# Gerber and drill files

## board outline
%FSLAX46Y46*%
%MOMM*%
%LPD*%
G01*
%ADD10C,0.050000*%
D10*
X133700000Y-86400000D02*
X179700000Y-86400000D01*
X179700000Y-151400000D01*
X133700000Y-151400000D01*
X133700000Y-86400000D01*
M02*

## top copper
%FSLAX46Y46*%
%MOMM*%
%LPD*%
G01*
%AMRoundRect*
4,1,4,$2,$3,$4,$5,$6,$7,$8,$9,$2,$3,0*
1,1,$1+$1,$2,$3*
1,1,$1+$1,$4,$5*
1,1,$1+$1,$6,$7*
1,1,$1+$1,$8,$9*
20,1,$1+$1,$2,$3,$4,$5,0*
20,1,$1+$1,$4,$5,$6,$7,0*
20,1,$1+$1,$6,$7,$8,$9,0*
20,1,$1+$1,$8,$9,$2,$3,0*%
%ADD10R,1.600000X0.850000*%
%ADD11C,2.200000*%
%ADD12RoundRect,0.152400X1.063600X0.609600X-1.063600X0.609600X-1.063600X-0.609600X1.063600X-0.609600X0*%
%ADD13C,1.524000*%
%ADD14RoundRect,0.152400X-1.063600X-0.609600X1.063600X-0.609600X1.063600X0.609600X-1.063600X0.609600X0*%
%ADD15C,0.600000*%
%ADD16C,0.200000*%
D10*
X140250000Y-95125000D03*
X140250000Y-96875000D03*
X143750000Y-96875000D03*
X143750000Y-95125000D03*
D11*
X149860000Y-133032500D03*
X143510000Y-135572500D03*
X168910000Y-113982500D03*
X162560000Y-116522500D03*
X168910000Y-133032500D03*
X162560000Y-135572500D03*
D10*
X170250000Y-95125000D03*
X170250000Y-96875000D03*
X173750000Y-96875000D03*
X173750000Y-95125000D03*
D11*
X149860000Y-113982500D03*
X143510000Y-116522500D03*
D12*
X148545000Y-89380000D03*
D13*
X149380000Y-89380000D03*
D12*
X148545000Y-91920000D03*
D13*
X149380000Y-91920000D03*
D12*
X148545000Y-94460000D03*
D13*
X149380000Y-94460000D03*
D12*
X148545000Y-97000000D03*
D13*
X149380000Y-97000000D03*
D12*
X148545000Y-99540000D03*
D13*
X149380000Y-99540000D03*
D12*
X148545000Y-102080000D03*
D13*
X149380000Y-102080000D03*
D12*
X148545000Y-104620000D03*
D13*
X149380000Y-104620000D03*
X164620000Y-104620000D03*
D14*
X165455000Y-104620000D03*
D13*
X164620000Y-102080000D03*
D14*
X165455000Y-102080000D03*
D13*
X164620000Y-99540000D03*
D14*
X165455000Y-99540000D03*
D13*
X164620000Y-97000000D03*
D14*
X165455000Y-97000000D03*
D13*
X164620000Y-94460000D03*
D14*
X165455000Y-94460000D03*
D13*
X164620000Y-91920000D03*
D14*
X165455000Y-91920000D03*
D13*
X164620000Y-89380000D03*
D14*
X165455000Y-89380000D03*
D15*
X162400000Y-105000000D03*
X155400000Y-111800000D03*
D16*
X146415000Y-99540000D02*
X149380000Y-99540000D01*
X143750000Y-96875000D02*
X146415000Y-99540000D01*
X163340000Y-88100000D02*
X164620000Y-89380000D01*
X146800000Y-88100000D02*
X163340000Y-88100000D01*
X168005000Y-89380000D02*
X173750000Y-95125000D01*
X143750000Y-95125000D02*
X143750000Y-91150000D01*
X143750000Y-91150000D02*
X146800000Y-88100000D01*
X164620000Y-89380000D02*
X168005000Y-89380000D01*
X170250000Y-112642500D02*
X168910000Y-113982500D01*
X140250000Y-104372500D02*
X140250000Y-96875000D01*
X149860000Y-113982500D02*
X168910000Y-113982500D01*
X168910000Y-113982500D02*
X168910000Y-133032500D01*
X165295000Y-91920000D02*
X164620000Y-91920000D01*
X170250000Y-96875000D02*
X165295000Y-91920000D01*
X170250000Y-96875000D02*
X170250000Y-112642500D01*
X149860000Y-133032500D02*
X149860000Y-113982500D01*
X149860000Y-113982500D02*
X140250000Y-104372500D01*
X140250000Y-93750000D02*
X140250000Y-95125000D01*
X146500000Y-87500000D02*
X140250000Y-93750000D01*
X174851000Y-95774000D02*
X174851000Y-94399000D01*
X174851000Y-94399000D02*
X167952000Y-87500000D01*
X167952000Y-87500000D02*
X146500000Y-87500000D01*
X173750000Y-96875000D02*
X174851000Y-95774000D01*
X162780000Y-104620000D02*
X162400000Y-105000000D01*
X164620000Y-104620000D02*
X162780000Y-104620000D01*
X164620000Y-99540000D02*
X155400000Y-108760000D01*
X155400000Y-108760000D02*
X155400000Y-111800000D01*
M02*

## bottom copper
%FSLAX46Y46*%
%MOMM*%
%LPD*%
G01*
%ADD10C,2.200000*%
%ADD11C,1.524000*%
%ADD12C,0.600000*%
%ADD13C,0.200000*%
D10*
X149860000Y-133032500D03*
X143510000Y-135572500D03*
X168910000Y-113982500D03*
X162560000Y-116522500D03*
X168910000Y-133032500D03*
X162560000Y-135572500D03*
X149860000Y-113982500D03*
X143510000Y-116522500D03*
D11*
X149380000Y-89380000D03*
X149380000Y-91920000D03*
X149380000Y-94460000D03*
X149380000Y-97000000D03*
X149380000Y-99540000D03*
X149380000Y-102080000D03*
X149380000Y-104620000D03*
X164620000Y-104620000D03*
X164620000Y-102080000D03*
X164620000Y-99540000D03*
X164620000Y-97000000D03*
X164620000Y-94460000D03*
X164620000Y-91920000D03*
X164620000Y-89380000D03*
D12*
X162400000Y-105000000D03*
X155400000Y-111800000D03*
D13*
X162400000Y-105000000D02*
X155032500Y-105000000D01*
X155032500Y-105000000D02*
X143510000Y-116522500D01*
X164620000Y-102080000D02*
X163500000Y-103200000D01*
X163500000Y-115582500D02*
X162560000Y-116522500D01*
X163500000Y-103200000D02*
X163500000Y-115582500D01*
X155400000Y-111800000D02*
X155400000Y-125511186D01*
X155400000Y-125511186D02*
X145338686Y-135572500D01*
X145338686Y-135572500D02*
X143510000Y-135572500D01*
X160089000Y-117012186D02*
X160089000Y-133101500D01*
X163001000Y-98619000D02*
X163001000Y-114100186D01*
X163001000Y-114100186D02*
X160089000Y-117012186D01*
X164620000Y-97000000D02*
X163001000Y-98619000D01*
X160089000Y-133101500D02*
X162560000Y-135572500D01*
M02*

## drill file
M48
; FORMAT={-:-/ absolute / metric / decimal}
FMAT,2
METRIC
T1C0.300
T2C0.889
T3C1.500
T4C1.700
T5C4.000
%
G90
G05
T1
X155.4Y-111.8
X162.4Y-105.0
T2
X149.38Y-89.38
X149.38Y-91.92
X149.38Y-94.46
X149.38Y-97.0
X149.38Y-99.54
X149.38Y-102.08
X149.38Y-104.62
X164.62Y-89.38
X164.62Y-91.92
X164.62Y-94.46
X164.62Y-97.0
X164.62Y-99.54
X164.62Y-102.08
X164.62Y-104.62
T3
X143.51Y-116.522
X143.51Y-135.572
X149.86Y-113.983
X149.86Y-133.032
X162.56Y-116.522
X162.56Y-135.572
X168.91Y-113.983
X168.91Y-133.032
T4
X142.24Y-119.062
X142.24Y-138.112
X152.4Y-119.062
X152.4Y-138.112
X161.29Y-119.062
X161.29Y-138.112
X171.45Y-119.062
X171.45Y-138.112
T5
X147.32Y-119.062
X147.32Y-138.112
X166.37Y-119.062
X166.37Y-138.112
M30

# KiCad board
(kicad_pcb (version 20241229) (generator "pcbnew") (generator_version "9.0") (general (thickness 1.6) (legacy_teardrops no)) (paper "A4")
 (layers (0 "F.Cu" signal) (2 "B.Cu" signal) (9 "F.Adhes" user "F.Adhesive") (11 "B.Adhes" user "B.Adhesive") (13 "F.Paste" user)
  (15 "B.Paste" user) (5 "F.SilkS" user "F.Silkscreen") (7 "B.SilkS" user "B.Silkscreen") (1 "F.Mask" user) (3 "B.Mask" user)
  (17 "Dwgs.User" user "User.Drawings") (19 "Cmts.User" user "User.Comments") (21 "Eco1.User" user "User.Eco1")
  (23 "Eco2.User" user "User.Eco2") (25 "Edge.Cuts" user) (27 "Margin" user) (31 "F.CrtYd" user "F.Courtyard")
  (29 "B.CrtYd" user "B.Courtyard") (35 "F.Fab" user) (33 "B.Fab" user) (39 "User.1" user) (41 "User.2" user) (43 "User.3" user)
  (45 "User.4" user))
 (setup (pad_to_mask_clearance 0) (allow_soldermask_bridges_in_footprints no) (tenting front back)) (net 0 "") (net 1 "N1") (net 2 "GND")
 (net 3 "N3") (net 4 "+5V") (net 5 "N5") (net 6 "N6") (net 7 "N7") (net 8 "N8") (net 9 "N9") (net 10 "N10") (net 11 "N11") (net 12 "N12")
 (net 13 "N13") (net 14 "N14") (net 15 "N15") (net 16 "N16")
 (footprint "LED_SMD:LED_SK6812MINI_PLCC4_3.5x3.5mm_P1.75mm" (layer "F.Cu") (at 142 96)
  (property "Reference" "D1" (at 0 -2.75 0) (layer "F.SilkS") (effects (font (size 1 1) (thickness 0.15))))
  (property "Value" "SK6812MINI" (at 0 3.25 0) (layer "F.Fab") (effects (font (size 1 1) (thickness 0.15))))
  (pad "1" smd rect (at -1.75 -0.875) (size 1.6 0.85) (layers "F.Cu" "F.Mask" "F.Paste") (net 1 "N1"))
  (pad "2" smd rect (at -1.75 0.875) (size 1.6 0.85) (layers "F.Cu" "F.Mask" "F.Paste") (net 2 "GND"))
  (pad "3" smd rect (at 1.75 0.875) (size 1.6 0.85) (layers "F.Cu" "F.Mask" "F.Paste") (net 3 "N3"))
  (pad "4" smd rect (at 1.75 -0.875) (size 1.6 0.85) (layers "F.Cu" "F.Mask" "F.Paste") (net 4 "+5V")))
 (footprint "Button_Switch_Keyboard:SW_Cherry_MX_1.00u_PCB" (layer "F.Cu") (at 149.86 133.0325)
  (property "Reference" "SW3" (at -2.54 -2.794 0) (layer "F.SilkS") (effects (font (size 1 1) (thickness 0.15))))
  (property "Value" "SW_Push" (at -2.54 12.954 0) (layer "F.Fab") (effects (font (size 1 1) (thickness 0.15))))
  (pad "" np_thru_hole circle (at -7.62 5.08) (size 1.7 1.7) (drill 1.7) (layers "*.Cu" "*.Mask"))
  (pad "" np_thru_hole circle (at -2.54 5.08) (size 4 4) (drill 4) (layers "*.Cu" "*.Mask"))
  (pad "" np_thru_hole circle (at 2.54 5.08) (size 1.7 1.7) (drill 1.7) (layers "*.Cu" "*.Mask"))
  (pad "1" thru_hole circle (at 0 0) (size 2.2 2.2) (drill 1.5) (layers "*.Cu" "*.Mask") (remove_unused_layers no) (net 2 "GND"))
  (pad "2" thru_hole circle (at -6.35 2.54) (size 2.2 2.2) (drill 1.5) (layers "*.Cu" "*.Mask") (remove_unused_layers no) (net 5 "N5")))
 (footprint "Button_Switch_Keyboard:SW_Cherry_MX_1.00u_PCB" (layer "F.Cu") (at 168.91 113.9825)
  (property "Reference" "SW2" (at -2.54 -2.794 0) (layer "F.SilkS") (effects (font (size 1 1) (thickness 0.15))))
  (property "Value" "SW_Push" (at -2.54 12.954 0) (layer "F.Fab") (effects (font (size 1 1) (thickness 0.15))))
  (pad "" np_thru_hole circle (at -7.62 5.08) (size 1.7 1.7) (drill 1.7) (layers "*.Cu" "*.Mask"))
  (pad "" np_thru_hole circle (at -2.54 5.08) (size 4 4) (drill 4) (layers "*.Cu" "*.Mask"))
  (pad "" np_thru_hole circle (at 2.54 5.08) (size 1.7 1.7) (drill 1.7) (layers "*.Cu" "*.Mask"))
  (pad "1" thru_hole circle (at 0 0) (size 2.2 2.2) (drill 1.5) (layers "*.Cu" "*.Mask") (remove_unused_layers no) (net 2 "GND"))
  (pad "2" thru_hole circle (at -6.35 2.54) (size 2.2 2.2) (drill 1.5) (layers "*.Cu" "*.Mask") (remove_unused_layers no) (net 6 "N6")))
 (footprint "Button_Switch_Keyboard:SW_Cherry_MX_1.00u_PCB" (layer "F.Cu") (at 168.91 133.0325)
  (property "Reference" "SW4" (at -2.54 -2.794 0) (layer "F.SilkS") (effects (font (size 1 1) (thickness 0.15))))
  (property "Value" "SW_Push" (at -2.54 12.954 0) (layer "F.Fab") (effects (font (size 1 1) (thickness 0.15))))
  (pad "" np_thru_hole circle (at -7.62 5.08) (size 1.7 1.7) (drill 1.7) (layers "*.Cu" "*.Mask"))
  (pad "" np_thru_hole circle (at -2.54 5.08) (size 4 4) (drill 4) (layers "*.Cu" "*.Mask"))
  (pad "" np_thru_hole circle (at 2.54 5.08) (size 1.7 1.7) (drill 1.7) (layers "*.Cu" "*.Mask"))
  (pad "1" thru_hole circle (at 0 0) (size 2.2 2.2) (drill 1.5) (layers "*.Cu" "*.Mask") (remove_unused_layers no) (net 2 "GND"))
  (pad "2" thru_hole circle (at -6.35 2.54) (size 2.2 2.2) (drill 1.5) (layers "*.Cu" "*.Mask") (remove_unused_layers no) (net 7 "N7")))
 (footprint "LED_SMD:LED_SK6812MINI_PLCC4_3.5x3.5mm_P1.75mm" (layer "F.Cu") (at 172 96)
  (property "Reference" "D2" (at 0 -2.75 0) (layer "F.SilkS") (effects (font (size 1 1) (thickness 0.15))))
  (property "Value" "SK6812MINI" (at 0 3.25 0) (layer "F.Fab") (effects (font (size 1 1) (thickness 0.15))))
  (pad "1" smd rect (at -1.75 -0.875) (size 1.6 0.85) (layers "F.Cu" "F.Mask" "F.Paste") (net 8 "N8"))
  (pad "2" smd rect (at -1.75 0.875) (size 1.6 0.85) (layers "F.Cu" "F.Mask" "F.Paste") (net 2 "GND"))
  (pad "3" smd rect (at 1.75 0.875) (size 1.6 0.85) (layers "F.Cu" "F.Mask" "F.Paste") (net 1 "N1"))
  (pad "4" smd rect (at 1.75 -0.875) (size 1.6 0.85) (layers "F.Cu" "F.Mask" "F.Paste") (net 4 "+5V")))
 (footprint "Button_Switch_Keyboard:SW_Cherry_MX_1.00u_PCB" (layer "F.Cu") (at 149.86 113.9825)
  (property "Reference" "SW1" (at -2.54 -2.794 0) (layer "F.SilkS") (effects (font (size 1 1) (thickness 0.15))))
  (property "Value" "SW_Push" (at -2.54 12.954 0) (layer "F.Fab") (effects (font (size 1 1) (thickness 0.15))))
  (pad "" np_thru_hole circle (at -7.62 5.08) (size 1.7 1.7) (drill 1.7) (layers "*.Cu" "*.Mask"))
  (pad "" np_thru_hole circle (at -2.54 5.08) (size 4 4) (drill 4) (layers "*.Cu" "*.Mask"))
  (pad "" np_thru_hole circle (at 2.54 5.08) (size 1.7 1.7) (drill 1.7) (layers "*.Cu" "*.Mask"))
  (pad "1" thru_hole circle (at 0 0) (size 2.2 2.2) (drill 1.5) (layers "*.Cu" "*.Mask") (remove_unused_layers no) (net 2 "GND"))
  (pad "2" thru_hole circle (at -6.35 2.54) (size 2.2 2.2) (drill 1.5) (layers "*.Cu" "*.Mask") (remove_unused_layers no) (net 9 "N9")))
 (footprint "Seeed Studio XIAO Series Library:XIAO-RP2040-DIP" (layer "F.Cu") (at 157 97)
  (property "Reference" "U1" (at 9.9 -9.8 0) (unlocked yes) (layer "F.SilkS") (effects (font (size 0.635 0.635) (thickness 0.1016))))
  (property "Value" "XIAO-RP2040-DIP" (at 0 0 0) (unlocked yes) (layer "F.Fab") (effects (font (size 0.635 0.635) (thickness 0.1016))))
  (pad "1" smd roundrect (at -8.455 -7.62 180) (size 2.432 1.524) (layers "F.Cu" "F.Mask") (roundrect_rratio 0.1) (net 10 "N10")
   (thermal_bridge_angle 45))
  (pad "1" thru_hole circle (at -7.62 -7.62 180) (size 1.524 1.524) (drill 0.889) (layers "*.Cu" "*.Mask") (remove_unused_layers no)
   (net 10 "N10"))
  (pad "2" smd roundrect (at -8.455 -5.08 180) (size 2.432 1.524) (layers "F.Cu" "F.Mask") (roundrect_rratio 0.1) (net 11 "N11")
   (thermal_bridge_angle 45))
  (pad "2" thru_hole circle (at -7.62 -5.08 180) (size 1.524 1.524) (drill 0.889) (layers "*.Cu" "*.Mask") (remove_unused_layers no)
   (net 11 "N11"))
  (pad "3" smd roundrect (at -8.455 -2.54 180) (size 2.432 1.524) (layers "F.Cu" "F.Mask") (roundrect_rratio 0.1) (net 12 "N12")
   (thermal_bridge_angle 45))
  (pad "3" thru_hole circle (at -7.62 -2.54 180) (size 1.524 1.524) (drill 0.889) (layers "*.Cu" "*.Mask") (remove_unused_layers no)
   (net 12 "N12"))
  (pad "4" smd roundrect (at -8.455 0 180) (size 2.432 1.524) (layers "F.Cu" "F.Mask") (roundrect_rratio 0.1) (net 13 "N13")
   (thermal_bridge_angle 45))
  (pad "4" thru_hole circle (at -7.62 0 180) (size 1.524 1.524) (drill 0.889) (layers "*.Cu" "*.Mask") (remove_unused_layers no)
   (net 13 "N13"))
  (pad "5" smd roundrect (at -8.455 2.54 180) (size 2.432 1.524) (layers "F.Cu" "F.Mask") (roundrect_rratio 0.1) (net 3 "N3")
   (thermal_bridge_angle 45))
  (pad "5" thru_hole circle (at -7.62 2.54 180) (size 1.524 1.524) (drill 0.889) (layers "*.Cu" "*.Mask") (remove_unused_layers no)
   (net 3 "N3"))
  (pad "6" smd roundrect (at -8.455 5.08 180) (size 2.432 1.524) (layers "F.Cu" "F.Mask") (roundrect_rratio 0.1) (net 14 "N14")
   (thermal_bridge_angle 45))
  (pad "6" thru_hole circle (at -7.62 5.08 180) (size 1.524 1.524) (drill 0.889) (layers "*.Cu" "*.Mask") (remove_unused_layers no)
   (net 14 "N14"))
  (pad "7" smd roundrect (at -8.455 7.62 180) (size 2.432 1.524) (layers "F.Cu" "F.Mask") (roundrect_rratio 0.1) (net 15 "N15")
   (thermal_bridge_angle 45))
  (pad "7" thru_hole circle (at -7.62 7.62 180) (size 1.524 1.524) (drill 0.889) (layers "*.Cu" "*.Mask") (remove_unused_layers no)
   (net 15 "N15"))
  (pad "8" thru_hole circle (at 7.62 7.62) (size 1.524 1.524) (drill 0.889) (layers "*.Cu" "*.Mask") (remove_unused_layers no) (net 9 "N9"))
  (pad "8" smd roundrect (at 8.455 7.62) (size 2.432 1.524) (layers "F.Cu" "F.Mask") (roundrect_rratio 0.1) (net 9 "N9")
   (thermal_bridge_angle 45))
  (pad "9" thru_hole circle (at 7.62 5.08) (size 1.524 1.524) (drill 0.889) (layers "*.Cu" "*.Mask") (remove_unused_layers no) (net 6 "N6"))
  (pad "9" smd roundrect (at 8.455 5.08) (size 2.432 1.524) (layers "F.Cu" "F.Mask") (roundrect_rratio 0.1) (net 6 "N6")
   (thermal_bridge_angle 45))
  (pad "10" thru_hole circle (at 7.62 2.54) (size 1.524 1.524) (drill 0.889) (layers "*.Cu" "*.Mask") (remove_unused_layers no) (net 5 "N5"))
  (pad "10" smd roundrect (at 8.455 2.54) (size 2.432 1.524) (layers "F.Cu" "F.Mask") (roundrect_rratio 0.1) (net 5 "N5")
   (thermal_bridge_angle 45))
  (pad "11" thru_hole circle (at 7.62 0) (size 1.524 1.524) (drill 0.889) (layers "*.Cu" "*.Mask") (remove_unused_layers no) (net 7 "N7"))
  (pad "11" smd roundrect (at 8.455 0) (size 2.432 1.524) (layers "F.Cu" "F.Mask") (roundrect_rratio 0.1) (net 7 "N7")
   (thermal_bridge_angle 45))
  (pad "12" thru_hole circle (at 7.62 -2.54) (size 1.524 1.524) (drill 0.889) (layers "*.Cu" "*.Mask") (remove_unused_layers no)
   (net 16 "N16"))
  (pad "12" smd roundrect (at 8.455 -2.54) (size 2.432 1.524) (layers "F.Cu" "F.Mask") (roundrect_rratio 0.1) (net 16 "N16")
   (thermal_bridge_angle 45))
  (pad "13" thru_hole circle (at 7.62 -5.08) (size 1.524 1.524) (drill 0.889) (layers "*.Cu" "*.Mask") (remove_unused_layers no)
   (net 2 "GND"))
  (pad "13" smd roundrect (at 8.455 -5.08) (size 2.432 1.524) (layers "F.Cu" "F.Mask") (roundrect_rratio 0.1) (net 2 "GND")
   (thermal_bridge_angle 45))
  (pad "14" thru_hole circle (at 7.62 -7.62) (size 1.524 1.524) (drill 0.889) (layers "*.Cu" "*.Mask") (remove_unused_layers no)
   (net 4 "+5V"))
  (pad "14" smd roundrect (at 8.455 -7.62) (size 2.432 1.524) (layers "F.Cu" "F.Mask") (roundrect_rratio 0.1) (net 4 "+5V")
   (thermal_bridge_angle 45)))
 (gr_rect (start 133.7 86.4) (end 179.7 151.4) (stroke (width 0.05) (type default)) (fill no) (layer "Edge.Cuts"))
 (segment (start 146.415 99.54) (end 149.38 99.54) (width 0.2) (layer "F.Cu") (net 3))
 (segment (start 143.75 96.875) (end 146.415 99.54) (width 0.2) (layer "F.Cu") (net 3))
 (segment (start 163.34 88.1) (end 164.62 89.38) (width 0.2) (layer "F.Cu") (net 4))
 (segment (start 146.8 88.1) (end 163.34 88.1) (width 0.2) (layer "F.Cu") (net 4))
 (segment (start 168.005 89.38) (end 173.75 95.125) (width 0.2) (layer "F.Cu") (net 4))
 (segment (start 143.75 95.125) (end 143.75 91.15) (width 0.2) (layer "F.Cu") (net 4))
 (segment (start 143.75 91.15) (end 146.8 88.1) (width 0.2) (layer "F.Cu") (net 4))
 (segment (start 164.62 89.38) (end 168.005 89.38) (width 0.2) (layer "F.Cu") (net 4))
 (segment (start 170.25 112.6425) (end 168.91 113.9825) (width 0.2) (layer "F.Cu") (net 2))
 (segment (start 140.25 104.3725) (end 140.25 96.875) (width 0.2) (layer "F.Cu") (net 2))
 (segment (start 149.86 113.9825) (end 168.91 113.9825) (width 0.2) (layer "F.Cu") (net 2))
 (segment (start 168.91 113.9825) (end 168.91 133.0325) (width 0.2) (layer "F.Cu") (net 2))
 (segment (start 165.295 91.92) (end 164.62 91.92) (width 0.2) (layer "F.Cu") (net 2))
 (segment (start 170.25 96.875) (end 165.295 91.92) (width 0.2) (layer "F.Cu") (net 2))
 (segment (start 170.25 96.875) (end 170.25 112.6425) (width 0.2) (layer "F.Cu") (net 2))
 (segment (start 149.86 133.0325) (end 149.86 113.9825) (width 0.2) (layer "F.Cu") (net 2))
 (segment (start 149.86 113.9825) (end 140.25 104.3725) (width 0.2) (layer "F.Cu") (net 2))
 (segment (start 140.25 93.75) (end 140.25 95.125) (width 0.2) (layer "F.Cu") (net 1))
 (segment (start 146.5 87.5) (end 140.25 93.75) (width 0.2) (layer "F.Cu") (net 1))
 (segment (start 174.851 95.774) (end 174.851 94.399) (width 0.2) (layer "F.Cu") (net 1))
 (segment (start 174.851 94.399) (end 167.952 87.5) (width 0.2) (layer "F.Cu") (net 1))
 (segment (start 167.952 87.5) (end 146.5 87.5) (width 0.2) (layer "F.Cu") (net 1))
 (segment (start 173.75 96.875) (end 174.851 95.774) (width 0.2) (layer "F.Cu") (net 1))
 (segment (start 162.78 104.62) (end 162.4 105) (width 0.2) (layer "F.Cu") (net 9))
 (segment (start 164.62 104.62) (end 162.78 104.62) (width 0.2) (layer "F.Cu") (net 9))
 (via (at 162.4 105) (size 0.6) (drill 0.3) (layers "F.Cu" "B.Cu") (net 9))
 (segment (start 162.4 105) (end 155.0325 105) (width 0.2) (layer "B.Cu") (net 9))
 (segment (start 155.0325 105) (end 143.51 116.5225) (width 0.2) (layer "B.Cu") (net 9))
 (segment (start 164.62 102.08) (end 163.5 103.2) (width 0.2) (layer "B.Cu") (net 6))
 (segment (start 163.5 115.5825) (end 162.56 116.5225) (width 0.2) (layer "B.Cu") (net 6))
 (segment (start 163.5 103.2) (end 163.5 115.5825) (width 0.2) (layer "B.Cu") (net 6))
 (segment (start 164.62 99.54) (end 155.4 108.76) (width 0.2) (layer "F.Cu") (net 5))
 (segment (start 155.4 108.76) (end 155.4 111.8) (width 0.2) (layer "F.Cu") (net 5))
 (via (at 155.4 111.8) (size 0.6) (drill 0.3) (layers "F.Cu" "B.Cu") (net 5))
 (segment (start 155.4 111.8) (end 155.4 125.511186) (width 0.2) (layer "B.Cu") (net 5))
 (segment (start 155.4 125.511186) (end 145.338686 135.5725) (width 0.2) (layer "B.Cu") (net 5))
 (segment (start 145.338686 135.5725) (end 143.51 135.5725) (width 0.2) (layer "B.Cu") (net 5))
 (segment (start 160.089 117.012186) (end 160.089 133.1015) (width 0.2) (layer "B.Cu") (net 7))
 (segment (start 163.001 98.619) (end 163.001 114.100186) (width 0.2) (layer "B.Cu") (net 7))
 (segment (start 163.001 114.100186) (end 160.089 117.012186) (width 0.2) (layer "B.Cu") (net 7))
 (segment (start 164.62 97) (end 163.001 98.619) (width 0.2) (layer "B.Cu") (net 7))
 (segment (start 160.089 133.1015) (end 162.56 135.5725) (width 0.2) (layer "B.Cu") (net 7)))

